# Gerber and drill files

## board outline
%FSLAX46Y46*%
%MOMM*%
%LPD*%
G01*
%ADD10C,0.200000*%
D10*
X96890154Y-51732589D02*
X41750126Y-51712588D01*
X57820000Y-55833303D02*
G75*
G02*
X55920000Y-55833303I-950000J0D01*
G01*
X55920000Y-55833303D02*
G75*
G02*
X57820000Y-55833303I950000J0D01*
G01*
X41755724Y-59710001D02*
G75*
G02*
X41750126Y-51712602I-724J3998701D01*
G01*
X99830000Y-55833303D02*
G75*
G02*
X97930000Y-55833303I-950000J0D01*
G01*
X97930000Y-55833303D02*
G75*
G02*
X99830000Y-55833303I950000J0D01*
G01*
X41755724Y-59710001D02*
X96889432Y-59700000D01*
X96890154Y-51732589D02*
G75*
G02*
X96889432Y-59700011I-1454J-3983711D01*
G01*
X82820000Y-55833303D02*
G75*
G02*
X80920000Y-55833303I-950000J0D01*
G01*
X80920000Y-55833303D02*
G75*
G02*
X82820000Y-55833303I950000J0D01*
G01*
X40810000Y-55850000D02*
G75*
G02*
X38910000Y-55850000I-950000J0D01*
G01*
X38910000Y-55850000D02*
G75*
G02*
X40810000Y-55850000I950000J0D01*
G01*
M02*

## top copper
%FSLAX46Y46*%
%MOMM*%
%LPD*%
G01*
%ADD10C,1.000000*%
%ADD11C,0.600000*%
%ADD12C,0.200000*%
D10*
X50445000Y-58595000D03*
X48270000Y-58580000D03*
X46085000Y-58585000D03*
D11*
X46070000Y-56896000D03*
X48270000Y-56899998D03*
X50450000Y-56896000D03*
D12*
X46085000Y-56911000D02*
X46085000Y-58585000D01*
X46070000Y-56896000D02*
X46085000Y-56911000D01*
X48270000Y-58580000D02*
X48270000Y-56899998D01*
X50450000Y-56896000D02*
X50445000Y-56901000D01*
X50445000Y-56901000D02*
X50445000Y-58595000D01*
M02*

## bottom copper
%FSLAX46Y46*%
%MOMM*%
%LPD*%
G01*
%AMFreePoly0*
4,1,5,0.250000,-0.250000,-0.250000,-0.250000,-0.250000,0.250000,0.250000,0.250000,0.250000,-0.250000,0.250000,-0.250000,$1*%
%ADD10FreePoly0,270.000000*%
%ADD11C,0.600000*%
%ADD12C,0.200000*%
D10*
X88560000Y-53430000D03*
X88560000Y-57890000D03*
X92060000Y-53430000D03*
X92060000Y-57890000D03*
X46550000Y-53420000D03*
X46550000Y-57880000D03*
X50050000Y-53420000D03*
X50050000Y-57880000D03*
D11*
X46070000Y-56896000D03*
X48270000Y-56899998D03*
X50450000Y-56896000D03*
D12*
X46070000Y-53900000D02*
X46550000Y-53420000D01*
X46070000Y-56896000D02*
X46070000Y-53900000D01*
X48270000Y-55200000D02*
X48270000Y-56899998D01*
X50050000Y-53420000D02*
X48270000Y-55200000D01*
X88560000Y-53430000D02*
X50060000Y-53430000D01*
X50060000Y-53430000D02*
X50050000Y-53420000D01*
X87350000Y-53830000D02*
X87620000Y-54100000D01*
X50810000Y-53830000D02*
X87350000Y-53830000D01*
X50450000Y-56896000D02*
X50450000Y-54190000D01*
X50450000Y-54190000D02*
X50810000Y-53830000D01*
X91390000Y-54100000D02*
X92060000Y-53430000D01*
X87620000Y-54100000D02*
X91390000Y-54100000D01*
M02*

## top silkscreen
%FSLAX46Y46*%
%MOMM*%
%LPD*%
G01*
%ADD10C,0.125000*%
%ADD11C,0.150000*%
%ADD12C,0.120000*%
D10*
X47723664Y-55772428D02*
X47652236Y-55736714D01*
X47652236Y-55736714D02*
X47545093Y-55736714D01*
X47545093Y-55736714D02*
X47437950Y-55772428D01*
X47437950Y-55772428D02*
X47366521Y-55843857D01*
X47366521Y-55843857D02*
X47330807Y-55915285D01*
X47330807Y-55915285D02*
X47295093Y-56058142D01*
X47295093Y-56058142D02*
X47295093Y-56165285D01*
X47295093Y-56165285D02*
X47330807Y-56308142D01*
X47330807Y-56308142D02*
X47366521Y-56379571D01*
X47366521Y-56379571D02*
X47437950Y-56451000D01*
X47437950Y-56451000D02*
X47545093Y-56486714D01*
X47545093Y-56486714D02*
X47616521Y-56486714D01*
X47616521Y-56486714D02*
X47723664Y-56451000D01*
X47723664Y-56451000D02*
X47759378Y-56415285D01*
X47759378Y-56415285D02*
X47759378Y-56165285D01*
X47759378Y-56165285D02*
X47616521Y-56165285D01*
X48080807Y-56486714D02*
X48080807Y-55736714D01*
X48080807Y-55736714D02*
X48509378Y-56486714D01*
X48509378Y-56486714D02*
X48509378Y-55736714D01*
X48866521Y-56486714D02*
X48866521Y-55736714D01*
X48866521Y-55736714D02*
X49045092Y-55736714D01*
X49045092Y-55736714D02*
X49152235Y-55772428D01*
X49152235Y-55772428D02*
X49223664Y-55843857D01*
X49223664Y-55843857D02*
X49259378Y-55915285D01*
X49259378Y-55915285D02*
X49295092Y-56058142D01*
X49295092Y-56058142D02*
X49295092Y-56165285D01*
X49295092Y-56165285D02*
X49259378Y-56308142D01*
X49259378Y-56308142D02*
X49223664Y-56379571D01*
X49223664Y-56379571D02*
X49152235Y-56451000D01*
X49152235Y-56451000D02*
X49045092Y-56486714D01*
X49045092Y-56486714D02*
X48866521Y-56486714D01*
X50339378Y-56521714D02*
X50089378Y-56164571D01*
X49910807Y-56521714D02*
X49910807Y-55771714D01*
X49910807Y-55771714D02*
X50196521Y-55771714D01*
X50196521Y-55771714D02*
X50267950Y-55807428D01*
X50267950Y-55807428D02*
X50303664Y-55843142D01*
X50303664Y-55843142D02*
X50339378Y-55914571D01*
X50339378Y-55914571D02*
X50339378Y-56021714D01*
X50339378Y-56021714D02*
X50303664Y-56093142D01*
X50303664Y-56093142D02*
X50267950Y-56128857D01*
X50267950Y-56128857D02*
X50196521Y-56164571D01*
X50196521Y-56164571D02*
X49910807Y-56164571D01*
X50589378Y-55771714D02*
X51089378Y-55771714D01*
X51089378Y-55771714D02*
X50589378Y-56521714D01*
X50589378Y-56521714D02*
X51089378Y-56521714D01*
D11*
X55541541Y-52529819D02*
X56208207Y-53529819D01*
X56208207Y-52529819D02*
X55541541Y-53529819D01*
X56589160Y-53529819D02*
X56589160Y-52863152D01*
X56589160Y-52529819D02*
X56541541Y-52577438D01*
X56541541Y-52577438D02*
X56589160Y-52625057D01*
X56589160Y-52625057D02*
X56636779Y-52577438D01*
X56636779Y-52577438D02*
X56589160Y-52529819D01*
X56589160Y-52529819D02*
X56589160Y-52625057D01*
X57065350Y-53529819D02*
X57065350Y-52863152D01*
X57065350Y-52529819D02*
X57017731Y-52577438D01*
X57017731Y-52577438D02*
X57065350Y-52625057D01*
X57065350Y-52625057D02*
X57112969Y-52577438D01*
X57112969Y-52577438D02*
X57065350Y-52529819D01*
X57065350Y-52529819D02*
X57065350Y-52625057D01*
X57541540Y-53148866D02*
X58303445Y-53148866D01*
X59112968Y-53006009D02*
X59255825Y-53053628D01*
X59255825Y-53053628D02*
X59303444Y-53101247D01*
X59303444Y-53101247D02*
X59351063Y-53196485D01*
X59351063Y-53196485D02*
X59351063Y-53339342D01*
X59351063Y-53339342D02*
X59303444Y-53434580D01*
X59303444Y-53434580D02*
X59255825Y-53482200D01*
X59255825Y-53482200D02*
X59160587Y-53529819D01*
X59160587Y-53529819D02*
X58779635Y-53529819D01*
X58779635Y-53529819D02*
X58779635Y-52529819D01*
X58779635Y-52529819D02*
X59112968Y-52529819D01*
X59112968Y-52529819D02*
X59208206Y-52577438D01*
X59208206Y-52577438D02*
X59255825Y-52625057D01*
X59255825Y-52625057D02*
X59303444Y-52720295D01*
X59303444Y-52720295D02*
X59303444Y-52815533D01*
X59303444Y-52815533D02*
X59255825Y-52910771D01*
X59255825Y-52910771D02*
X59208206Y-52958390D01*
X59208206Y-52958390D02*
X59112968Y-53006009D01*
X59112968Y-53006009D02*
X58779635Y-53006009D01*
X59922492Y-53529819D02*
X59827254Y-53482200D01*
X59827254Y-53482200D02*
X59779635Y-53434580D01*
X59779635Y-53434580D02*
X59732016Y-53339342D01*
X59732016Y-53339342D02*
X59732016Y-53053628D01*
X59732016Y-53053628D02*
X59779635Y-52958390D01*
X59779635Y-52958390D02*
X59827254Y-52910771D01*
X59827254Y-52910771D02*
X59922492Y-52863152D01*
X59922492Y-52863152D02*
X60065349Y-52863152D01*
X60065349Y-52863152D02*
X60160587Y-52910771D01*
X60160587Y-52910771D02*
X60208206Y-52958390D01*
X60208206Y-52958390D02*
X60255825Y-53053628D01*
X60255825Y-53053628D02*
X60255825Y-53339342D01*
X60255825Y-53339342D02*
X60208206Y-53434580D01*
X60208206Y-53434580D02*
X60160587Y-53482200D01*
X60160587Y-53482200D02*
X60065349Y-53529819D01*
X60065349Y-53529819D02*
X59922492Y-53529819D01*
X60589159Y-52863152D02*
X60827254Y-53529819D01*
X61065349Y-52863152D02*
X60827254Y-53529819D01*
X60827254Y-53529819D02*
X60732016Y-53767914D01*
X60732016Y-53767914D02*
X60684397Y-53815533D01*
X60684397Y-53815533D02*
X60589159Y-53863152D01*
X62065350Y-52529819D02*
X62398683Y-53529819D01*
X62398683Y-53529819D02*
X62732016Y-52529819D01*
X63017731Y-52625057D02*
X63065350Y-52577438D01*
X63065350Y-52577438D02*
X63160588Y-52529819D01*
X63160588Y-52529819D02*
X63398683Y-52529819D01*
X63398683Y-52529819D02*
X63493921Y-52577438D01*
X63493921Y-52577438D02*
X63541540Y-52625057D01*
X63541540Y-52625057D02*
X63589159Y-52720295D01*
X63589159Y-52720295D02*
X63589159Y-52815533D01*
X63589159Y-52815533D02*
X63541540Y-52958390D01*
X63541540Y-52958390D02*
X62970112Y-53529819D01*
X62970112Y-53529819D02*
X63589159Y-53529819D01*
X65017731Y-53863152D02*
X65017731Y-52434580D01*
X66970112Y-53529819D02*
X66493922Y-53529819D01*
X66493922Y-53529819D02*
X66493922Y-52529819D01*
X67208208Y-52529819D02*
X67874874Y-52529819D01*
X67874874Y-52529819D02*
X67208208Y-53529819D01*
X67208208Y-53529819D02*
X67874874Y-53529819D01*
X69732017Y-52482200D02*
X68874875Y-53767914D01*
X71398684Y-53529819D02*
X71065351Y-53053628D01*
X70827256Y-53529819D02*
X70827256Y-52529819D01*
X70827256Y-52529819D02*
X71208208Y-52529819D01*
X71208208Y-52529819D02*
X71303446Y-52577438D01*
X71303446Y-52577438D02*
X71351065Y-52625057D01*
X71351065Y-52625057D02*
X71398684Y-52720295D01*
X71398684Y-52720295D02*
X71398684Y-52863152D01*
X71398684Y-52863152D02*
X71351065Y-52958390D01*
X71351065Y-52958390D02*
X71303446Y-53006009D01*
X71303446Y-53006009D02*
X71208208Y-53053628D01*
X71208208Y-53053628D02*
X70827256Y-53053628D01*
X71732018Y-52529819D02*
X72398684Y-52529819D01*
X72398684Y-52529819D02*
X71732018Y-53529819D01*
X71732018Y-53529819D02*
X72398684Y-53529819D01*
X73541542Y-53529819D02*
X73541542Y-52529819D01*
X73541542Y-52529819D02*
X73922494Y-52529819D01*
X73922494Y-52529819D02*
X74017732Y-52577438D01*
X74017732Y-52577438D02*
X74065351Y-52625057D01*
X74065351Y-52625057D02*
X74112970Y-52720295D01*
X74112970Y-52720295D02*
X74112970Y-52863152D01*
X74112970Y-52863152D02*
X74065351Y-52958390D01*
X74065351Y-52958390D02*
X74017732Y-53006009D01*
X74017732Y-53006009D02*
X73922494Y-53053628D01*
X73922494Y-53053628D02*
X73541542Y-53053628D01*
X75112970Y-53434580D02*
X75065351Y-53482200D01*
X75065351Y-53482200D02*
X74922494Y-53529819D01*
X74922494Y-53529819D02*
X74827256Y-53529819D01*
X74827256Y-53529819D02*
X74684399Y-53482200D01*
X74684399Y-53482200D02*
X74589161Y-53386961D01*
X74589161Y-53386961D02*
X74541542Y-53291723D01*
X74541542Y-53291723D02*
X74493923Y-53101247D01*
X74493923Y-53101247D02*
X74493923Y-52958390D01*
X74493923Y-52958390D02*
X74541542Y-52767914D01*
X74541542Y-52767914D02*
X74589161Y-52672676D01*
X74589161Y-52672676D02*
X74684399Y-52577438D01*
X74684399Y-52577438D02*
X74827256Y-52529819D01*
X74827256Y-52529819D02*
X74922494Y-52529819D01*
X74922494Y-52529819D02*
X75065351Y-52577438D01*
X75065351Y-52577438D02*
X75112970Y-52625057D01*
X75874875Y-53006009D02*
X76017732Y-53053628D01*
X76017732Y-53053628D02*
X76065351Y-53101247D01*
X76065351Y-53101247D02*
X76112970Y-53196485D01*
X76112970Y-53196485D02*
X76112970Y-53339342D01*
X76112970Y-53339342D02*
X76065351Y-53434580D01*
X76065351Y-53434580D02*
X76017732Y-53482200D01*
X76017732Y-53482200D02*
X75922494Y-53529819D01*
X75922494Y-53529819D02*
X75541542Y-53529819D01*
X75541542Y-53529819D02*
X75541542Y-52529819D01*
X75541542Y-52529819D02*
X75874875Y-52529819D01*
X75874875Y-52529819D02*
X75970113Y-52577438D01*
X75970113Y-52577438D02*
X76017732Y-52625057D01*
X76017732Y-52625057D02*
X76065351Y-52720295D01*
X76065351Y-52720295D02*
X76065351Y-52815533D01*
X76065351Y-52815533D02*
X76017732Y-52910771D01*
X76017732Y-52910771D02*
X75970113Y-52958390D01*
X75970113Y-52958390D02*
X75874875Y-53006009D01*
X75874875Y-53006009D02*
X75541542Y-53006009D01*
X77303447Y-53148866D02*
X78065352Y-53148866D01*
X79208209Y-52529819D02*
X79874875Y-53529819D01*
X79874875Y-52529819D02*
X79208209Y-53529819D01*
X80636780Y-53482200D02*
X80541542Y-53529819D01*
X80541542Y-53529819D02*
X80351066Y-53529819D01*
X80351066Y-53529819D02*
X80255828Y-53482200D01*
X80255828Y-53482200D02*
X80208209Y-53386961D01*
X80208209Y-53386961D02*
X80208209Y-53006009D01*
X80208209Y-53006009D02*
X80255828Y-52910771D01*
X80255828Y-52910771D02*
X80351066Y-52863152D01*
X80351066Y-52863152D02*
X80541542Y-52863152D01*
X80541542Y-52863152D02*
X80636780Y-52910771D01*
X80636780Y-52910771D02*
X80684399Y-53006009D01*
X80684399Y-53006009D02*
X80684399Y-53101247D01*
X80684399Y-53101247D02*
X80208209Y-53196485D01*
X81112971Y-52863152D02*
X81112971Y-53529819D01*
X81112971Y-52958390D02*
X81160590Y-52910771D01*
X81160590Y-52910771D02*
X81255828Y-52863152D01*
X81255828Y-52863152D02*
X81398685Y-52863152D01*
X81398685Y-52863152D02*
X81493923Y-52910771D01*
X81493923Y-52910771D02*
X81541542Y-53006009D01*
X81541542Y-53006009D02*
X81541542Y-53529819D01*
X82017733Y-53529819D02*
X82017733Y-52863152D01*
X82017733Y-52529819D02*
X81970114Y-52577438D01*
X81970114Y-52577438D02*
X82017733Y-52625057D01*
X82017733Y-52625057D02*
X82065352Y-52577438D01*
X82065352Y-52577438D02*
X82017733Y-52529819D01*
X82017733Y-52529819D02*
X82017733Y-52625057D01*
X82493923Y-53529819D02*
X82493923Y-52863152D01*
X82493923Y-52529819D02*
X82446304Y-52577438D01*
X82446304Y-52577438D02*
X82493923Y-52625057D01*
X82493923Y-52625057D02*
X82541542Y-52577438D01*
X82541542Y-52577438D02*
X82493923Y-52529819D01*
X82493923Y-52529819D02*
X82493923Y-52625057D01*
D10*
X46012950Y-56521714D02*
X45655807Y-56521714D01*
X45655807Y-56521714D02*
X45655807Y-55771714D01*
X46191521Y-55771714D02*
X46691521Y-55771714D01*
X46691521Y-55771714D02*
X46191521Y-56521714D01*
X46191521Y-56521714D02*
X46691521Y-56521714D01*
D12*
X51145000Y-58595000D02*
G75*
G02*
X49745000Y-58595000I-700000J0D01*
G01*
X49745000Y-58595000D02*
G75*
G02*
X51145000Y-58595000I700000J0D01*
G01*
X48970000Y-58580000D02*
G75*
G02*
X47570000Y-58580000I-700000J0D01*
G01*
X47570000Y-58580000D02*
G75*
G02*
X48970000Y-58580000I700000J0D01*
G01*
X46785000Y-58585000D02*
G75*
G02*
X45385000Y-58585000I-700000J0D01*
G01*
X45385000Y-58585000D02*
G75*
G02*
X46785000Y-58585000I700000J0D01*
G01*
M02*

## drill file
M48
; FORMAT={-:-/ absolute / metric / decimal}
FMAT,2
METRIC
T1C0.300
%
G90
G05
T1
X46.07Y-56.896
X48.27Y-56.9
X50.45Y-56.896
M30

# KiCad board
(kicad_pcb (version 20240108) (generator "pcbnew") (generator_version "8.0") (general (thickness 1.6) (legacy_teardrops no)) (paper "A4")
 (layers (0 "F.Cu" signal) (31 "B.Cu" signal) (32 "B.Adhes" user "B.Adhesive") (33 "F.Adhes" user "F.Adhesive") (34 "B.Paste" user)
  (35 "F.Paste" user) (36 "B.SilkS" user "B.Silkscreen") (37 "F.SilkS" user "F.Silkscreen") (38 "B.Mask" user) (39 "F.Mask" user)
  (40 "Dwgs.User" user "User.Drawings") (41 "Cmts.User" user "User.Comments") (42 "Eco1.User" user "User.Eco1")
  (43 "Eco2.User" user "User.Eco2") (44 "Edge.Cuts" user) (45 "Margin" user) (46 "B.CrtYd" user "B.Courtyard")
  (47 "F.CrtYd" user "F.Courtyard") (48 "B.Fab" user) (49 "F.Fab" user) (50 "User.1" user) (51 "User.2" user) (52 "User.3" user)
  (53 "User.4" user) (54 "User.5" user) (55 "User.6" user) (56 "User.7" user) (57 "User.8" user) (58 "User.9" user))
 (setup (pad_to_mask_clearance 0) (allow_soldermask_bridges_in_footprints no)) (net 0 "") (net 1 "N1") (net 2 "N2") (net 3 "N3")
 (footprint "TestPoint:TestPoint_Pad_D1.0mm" (layer "F.Cu") (at 50.445 58.595)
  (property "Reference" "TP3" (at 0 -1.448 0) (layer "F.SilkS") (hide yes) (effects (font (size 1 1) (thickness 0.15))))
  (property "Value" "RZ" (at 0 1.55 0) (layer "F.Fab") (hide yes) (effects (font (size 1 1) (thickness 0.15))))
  (fp_circle (center 0 0) (end 0 0.7) (stroke (width 0.12) (type solid)) (fill none) (layer "F.SilkS"))
  (pad "1" smd circle (at 0 0) (size 1 1) (layers "F.Cu" "F.Mask") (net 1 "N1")))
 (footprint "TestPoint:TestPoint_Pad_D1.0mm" (layer "F.Cu") (at 48.27 58.58)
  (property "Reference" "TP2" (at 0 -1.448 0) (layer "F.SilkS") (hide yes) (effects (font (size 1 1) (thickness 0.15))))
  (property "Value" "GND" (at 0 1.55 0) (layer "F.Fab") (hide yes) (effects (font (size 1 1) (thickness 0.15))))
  (fp_circle (center 0 0) (end 0 0.7) (stroke (width 0.12) (type solid)) (fill none) (layer "F.SilkS"))
  (pad "1" smd circle (at 0 0) (size 1 1) (layers "F.Cu" "F.Mask") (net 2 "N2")))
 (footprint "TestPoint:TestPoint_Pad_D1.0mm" (layer "F.Cu") (at 46.085 58.585)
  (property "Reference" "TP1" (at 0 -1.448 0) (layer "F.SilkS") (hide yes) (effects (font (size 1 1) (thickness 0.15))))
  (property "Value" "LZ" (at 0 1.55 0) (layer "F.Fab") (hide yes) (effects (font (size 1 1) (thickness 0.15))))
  (fp_circle (center 0 0) (end 0 0.7) (stroke (width 0.12) (type solid)) (fill none) (layer "F.SilkS"))
  (pad "1" smd circle (at 0 0) (size 1 1) (layers "F.Cu" "F.Mask") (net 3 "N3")))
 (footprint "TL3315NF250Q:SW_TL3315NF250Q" (layer "B.Cu") (at 90.31 55.66 -90)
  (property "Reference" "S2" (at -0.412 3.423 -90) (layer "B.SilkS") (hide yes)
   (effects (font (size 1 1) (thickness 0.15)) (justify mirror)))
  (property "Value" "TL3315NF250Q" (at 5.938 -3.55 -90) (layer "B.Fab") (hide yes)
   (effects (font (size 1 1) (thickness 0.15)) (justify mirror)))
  (pad "1" smd custom (at -2.23 1.75 270) (size 0.5 0.5) (layers "B.Cu") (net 2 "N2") (options (clearance outline) (anchor rect))
   (primitives))
  (pad "2" smd custom (at 2.23 1.75 270) (size 0.5 0.5) (layers "B.Cu") (options (clearance outline) (anchor rect)) (primitives))
  (pad "3" smd custom (at -2.23 -1.75 270) (size 0.5 0.5) (layers "B.Cu") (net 1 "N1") (options (clearance outline) (anchor rect))
   (primitives))
  (pad "4" smd custom (at 2.23 -1.75 270) (size 0.5 0.5) (layers "B.Cu") (options (clearance outline) (anchor rect)) (primitives)))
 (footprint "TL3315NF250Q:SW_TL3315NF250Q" (layer "B.Cu") (at 48.3 55.65 -90)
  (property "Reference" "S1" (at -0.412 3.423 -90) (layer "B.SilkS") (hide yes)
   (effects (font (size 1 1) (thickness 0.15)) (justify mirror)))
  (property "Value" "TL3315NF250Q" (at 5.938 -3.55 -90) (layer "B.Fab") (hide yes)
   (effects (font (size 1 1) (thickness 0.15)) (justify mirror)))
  (pad "1" smd custom (at -2.23 1.75 270) (size 0.5 0.5) (layers "B.Cu") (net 3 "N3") (options (clearance outline) (anchor rect))
   (primitives))
  (pad "2" smd custom (at 2.23 1.75 270) (size 0.5 0.5) (layers "B.Cu") (options (clearance outline) (anchor rect)) (primitives))
  (pad "3" smd custom (at -2.23 -1.75 270) (size 0.5 0.5) (layers "B.Cu") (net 2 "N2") (options (clearance outline) (anchor rect))
   (primitives))
  (pad "4" smd custom (at 2.23 -1.75 270) (size 0.5 0.5) (layers "B.Cu") (options (clearance outline) (anchor rect)) (primitives)))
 (gr_line (start 96.890154 51.732589) (end 41.750126 51.712588) (stroke (width 0.2) (type default)) (layer "Edge.Cuts"))
 (gr_circle (center 56.87 55.833303) (end 56.87 54.883303) (stroke (width 0.2) (type default)) (fill none) (layer "Edge.Cuts"))
 (gr_arc (start 41.755724 59.710001) (mid 37.756293 55.714093) (end 41.750126 51.712588) (stroke (width 0.2) (type default))
  (layer "Edge.Cuts"))
 (gr_circle (center 98.88 55.833303) (end 98.88 54.883303) (stroke (width 0.2) (type default)) (fill none) (layer "Edge.Cuts"))
 (gr_line (start 41.755724 59.710001) (end 96.889432 59.7) (stroke (width 0.2) (type default)) (layer "Edge.Cuts"))
 (gr_arc (start 96.890154 51.732589) (mid 100.872414 55.716655) (end 96.889432 59.7) (stroke (width 0.2) (type default)) (layer "Edge.Cuts"))
 (gr_circle (center 81.87 55.833303) (end 81.87 54.883303) (stroke (width 0.2) (type default)) (fill none) (layer "Edge.Cuts"))
 (gr_circle (center 39.86 55.85) (end 39.86 54.9) (stroke (width 0.2) (type default)) (fill none) (layer "Edge.Cuts"))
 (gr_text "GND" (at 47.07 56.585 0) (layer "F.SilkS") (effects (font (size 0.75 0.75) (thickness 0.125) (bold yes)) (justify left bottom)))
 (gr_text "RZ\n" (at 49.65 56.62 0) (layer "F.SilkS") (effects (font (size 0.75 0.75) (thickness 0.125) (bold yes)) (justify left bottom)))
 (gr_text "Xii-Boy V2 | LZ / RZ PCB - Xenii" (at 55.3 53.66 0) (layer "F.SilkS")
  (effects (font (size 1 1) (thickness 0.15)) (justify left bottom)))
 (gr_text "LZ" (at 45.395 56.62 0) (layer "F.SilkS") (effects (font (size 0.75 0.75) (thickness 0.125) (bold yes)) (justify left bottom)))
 (segment (start 46.085 56.911) (end 46.085 58.585) (width 0.2) (layer "F.Cu") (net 3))
 (segment (start 46.07 56.896) (end 46.085 56.911) (width 0.2) (layer "F.Cu") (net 3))
 (via (at 46.07 56.896) (size 0.6) (drill 0.3) (layers "F.Cu" "B.Cu") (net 3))
 (segment (start 46.07 53.9) (end 46.55 53.42) (width 0.2) (layer "B.Cu") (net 3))
 (segment (start 46.07 56.896) (end 46.07 53.9) (width 0.2) (layer "B.Cu") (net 3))
 (segment (start 48.27 58.58) (end 48.27 56.899998) (width 0.2) (layer "F.Cu") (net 2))
 (via (at 48.27 56.899998) (size 0.6) (drill 0.3) (layers "F.Cu" "B.Cu") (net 2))
 (segment (start 48.27 55.2) (end 48.27 56.899998) (width 0.2) (layer "B.Cu") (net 2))
 (segment (start 50.05 53.42) (end 48.27 55.2) (width 0.2) (layer "B.Cu") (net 2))
 (segment (start 88.56 53.43) (end 50.06 53.43) (width 0.2) (layer "B.Cu") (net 2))
 (segment (start 50.06 53.43) (end 50.05 53.42) (width 0.2) (layer "B.Cu") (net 2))
 (segment (start 50.45 56.896) (end 50.445 56.901) (width 0.2) (layer "F.Cu") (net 1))
 (segment (start 50.445 56.901) (end 50.445 58.595) (width 0.2) (layer "F.Cu") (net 1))
 (via (at 50.45 56.896) (size 0.6) (drill 0.3) (layers "F.Cu" "B.Cu") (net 1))
 (segment (start 87.35 53.83) (end 87.62 54.1) (width 0.2) (layer "B.Cu") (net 1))
 (segment (start 50.81 53.83) (end 87.35 53.83) (width 0.2) (layer "B.Cu") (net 1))
 (segment (start 50.45 56.896) (end 50.45 54.19) (width 0.2) (layer "B.Cu") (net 1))
 (segment (start 50.45 54.19) (end 50.81 53.83) (width 0.2) (layer "B.Cu") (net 1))
 (segment (start 91.39 54.1) (end 92.06 53.43) (width 0.2) (layer "B.Cu") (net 1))
 (segment (start 87.62 54.1) (end 91.39 54.1) (width 0.2) (layer "B.Cu") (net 1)))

